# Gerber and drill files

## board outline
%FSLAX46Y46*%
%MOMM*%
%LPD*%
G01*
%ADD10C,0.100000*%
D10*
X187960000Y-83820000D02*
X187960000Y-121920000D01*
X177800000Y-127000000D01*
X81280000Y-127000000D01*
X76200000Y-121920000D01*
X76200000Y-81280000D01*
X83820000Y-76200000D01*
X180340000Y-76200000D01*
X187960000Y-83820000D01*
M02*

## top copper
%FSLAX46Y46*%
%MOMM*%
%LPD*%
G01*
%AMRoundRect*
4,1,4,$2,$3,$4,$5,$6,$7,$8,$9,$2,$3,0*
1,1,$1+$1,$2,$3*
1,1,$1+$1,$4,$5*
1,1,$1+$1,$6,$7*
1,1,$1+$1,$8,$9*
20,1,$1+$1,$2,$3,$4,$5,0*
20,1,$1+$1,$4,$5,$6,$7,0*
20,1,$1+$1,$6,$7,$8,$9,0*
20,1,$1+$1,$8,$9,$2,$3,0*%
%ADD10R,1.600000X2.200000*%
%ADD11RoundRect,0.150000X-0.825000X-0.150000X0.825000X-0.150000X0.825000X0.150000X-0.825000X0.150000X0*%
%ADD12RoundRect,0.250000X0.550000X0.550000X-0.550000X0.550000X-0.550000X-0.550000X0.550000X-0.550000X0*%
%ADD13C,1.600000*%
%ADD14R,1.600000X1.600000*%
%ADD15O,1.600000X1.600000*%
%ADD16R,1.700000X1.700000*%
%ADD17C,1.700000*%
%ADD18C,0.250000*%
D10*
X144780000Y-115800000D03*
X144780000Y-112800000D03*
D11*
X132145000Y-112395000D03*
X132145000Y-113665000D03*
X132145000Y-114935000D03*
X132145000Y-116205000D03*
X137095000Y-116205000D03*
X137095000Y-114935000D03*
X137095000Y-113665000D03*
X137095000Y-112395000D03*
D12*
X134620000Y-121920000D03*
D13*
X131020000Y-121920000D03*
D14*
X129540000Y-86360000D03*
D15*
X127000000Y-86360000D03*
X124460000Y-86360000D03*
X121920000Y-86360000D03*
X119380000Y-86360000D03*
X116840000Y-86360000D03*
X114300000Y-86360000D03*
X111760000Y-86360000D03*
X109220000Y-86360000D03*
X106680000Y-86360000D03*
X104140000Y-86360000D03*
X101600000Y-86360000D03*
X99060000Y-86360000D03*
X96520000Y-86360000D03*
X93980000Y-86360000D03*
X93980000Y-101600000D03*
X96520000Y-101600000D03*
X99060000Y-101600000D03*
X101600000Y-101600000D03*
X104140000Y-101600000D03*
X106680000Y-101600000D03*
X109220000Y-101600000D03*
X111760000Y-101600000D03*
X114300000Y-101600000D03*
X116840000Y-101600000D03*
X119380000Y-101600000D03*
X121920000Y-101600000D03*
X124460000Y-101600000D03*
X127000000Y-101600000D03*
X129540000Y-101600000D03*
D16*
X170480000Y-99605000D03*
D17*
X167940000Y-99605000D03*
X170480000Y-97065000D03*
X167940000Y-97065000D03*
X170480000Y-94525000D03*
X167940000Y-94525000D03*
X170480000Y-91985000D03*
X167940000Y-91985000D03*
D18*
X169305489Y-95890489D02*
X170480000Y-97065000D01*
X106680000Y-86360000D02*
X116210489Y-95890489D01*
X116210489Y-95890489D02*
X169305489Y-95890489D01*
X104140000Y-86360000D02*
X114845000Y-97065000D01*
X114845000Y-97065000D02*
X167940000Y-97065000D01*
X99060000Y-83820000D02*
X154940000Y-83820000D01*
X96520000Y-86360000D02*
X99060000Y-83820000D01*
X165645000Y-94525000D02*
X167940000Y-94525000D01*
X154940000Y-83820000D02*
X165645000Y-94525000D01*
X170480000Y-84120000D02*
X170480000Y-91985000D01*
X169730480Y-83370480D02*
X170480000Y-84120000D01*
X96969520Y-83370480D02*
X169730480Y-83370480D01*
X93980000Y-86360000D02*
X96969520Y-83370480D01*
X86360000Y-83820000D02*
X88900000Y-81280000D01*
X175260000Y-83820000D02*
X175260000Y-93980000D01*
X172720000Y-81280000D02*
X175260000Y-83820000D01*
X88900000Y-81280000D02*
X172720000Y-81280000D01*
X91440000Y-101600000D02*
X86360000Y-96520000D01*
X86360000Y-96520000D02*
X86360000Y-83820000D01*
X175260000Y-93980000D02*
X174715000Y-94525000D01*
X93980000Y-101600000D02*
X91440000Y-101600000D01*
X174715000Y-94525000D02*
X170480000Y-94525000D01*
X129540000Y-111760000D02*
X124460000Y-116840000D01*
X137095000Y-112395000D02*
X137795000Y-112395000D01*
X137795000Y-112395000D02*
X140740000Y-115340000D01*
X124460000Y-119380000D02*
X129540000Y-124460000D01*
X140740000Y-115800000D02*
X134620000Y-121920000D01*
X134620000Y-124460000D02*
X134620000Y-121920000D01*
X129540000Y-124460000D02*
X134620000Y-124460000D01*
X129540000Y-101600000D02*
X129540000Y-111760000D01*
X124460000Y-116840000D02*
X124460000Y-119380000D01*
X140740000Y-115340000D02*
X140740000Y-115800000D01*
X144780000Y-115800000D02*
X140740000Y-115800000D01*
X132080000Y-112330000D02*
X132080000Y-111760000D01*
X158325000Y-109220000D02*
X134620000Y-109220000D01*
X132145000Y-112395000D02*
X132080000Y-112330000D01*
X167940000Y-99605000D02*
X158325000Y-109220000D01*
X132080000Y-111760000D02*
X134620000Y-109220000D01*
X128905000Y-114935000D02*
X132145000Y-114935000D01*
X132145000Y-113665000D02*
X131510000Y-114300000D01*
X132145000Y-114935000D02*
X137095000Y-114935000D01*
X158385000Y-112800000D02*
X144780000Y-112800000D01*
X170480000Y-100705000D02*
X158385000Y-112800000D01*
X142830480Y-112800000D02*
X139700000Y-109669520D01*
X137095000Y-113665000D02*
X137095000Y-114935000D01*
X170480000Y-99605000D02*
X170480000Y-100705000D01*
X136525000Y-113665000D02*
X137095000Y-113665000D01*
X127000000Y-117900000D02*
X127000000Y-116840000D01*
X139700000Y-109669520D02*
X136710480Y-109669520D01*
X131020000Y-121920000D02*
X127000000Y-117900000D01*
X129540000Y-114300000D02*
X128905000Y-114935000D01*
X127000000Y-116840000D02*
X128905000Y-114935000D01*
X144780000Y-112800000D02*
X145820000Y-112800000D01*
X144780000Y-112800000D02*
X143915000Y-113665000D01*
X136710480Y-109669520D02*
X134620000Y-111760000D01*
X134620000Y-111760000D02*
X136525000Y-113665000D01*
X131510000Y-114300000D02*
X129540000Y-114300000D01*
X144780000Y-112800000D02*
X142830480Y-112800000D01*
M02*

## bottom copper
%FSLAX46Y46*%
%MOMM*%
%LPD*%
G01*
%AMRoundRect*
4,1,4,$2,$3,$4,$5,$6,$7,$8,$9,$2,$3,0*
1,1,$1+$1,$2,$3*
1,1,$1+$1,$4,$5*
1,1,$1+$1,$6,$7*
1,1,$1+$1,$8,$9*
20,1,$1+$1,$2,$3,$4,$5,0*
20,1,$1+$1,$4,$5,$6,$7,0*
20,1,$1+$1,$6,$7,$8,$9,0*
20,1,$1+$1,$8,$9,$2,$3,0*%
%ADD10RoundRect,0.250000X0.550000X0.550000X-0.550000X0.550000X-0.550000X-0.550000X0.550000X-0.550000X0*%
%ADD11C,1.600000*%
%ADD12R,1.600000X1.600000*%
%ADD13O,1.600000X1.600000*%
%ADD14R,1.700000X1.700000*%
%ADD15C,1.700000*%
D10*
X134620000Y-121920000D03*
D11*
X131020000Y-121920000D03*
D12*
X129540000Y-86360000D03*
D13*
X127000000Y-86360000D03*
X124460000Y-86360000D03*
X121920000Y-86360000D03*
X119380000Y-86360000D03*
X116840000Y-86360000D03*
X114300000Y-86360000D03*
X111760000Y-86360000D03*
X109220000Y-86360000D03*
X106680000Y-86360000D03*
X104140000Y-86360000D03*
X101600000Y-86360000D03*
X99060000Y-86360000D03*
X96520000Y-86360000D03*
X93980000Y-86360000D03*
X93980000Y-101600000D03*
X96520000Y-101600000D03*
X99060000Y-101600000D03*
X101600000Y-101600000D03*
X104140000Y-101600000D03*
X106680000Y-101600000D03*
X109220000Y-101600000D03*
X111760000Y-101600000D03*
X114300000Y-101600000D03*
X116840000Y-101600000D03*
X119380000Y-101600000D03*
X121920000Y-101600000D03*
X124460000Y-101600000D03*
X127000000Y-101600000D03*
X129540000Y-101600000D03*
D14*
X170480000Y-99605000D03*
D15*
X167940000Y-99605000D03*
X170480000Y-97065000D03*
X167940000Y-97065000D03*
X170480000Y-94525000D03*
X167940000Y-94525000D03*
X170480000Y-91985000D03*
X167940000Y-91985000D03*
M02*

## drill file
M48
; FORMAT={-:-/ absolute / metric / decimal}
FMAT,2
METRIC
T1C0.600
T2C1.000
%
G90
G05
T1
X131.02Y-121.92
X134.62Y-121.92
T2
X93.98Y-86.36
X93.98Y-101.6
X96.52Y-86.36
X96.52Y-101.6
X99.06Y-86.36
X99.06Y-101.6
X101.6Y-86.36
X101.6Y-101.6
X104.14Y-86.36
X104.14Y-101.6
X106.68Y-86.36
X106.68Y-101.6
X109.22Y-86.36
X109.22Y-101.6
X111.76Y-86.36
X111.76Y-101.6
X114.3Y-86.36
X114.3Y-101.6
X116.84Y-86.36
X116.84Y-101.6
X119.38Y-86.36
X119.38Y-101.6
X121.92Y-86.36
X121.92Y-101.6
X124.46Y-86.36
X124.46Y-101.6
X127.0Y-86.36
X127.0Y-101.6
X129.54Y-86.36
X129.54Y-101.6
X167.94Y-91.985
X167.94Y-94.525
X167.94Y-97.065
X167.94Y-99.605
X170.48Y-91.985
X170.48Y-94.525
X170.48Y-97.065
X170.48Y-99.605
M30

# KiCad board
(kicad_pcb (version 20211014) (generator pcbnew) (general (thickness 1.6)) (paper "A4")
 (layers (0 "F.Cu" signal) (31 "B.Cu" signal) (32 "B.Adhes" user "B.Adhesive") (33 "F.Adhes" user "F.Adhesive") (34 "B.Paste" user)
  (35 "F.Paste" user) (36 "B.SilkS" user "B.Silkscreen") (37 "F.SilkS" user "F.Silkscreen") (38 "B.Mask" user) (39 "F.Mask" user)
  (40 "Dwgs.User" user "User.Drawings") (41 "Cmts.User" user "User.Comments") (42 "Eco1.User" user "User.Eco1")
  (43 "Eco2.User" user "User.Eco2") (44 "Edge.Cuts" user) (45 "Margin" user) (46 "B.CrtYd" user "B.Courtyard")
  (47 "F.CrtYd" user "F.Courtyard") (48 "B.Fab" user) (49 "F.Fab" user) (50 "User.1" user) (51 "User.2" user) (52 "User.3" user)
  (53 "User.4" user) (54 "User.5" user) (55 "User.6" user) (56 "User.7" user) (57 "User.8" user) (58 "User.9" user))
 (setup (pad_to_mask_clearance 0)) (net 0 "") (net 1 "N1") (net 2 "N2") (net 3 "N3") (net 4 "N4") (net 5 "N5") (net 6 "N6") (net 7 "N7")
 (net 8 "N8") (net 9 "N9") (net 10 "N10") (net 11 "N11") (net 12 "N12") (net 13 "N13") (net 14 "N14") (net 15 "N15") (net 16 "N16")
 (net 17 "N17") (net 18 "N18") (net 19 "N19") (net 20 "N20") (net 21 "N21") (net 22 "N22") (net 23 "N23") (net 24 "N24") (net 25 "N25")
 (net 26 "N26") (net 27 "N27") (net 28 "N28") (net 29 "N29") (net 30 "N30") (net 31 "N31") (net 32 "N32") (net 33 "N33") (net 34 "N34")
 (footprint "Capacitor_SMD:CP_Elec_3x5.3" (layer "F.Cu") (at 144.78 114.3 90)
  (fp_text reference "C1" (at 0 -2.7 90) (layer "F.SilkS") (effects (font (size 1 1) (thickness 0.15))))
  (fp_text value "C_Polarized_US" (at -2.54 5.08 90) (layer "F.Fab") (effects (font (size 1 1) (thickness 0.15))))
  (pad "1" smd rect (at -1.5 0 90) (size 2.2 1.6) (layers "F.Cu" "F.Paste" "F.Mask") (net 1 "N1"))
  (pad "2" smd rect (at 1.5 0 90) (size 2.2 1.6) (layers "F.Cu" "F.Paste" "F.Mask") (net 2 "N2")))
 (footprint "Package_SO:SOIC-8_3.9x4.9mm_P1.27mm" (layer "F.Cu") (at 134.62 114.3)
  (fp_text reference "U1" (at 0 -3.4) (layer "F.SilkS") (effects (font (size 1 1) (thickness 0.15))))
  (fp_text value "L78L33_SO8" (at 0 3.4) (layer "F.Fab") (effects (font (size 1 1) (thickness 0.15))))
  (pad "1" smd roundrect (at -2.475 -1.905) (size 1.95 0.6) (layers "F.Cu" "F.Paste" "F.Mask") (roundrect_rratio 0.25) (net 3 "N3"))
  (pad "2" smd roundrect (at -2.475 -0.635) (size 1.95 0.6) (layers "F.Cu" "F.Paste" "F.Mask") (roundrect_rratio 0.25) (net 2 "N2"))
  (pad "3" smd roundrect (at -2.475 0.635) (size 1.95 0.6) (layers "F.Cu" "F.Paste" "F.Mask") (roundrect_rratio 0.25) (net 2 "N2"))
  (pad "4" smd roundrect (at -2.475 1.905) (size 1.95 0.6) (layers "F.Cu" "F.Paste" "F.Mask") (roundrect_rratio 0.25) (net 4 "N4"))
  (pad "5" smd roundrect (at 2.475 1.905) (size 1.95 0.6) (layers "F.Cu" "F.Paste" "F.Mask") (roundrect_rratio 0.25) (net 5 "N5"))
  (pad "6" smd roundrect (at 2.475 0.635) (size 1.95 0.6) (layers "F.Cu" "F.Paste" "F.Mask") (roundrect_rratio 0.25) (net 2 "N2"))
  (pad "7" smd roundrect (at 2.475 -0.635) (size 1.95 0.6) (layers "F.Cu" "F.Paste" "F.Mask") (roundrect_rratio 0.25) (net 2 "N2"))
  (pad "8" smd roundrect (at 2.475 -1.905) (size 1.95 0.6) (layers "F.Cu" "F.Paste" "F.Mask") (roundrect_rratio 0.25) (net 1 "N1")))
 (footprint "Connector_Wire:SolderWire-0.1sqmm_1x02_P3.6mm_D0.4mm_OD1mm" (layer "F.Cu") (at 134.62 121.92 180)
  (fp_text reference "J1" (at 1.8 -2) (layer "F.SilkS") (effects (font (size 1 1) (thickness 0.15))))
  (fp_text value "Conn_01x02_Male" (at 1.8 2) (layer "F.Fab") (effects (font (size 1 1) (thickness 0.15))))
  (pad "1" thru_hole roundrect (at 0 0 180) (size 1.6 1.6) (drill 0.6) (layers *.Cu *.Mask) (roundrect_rratio 0.15625) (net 1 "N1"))
  (pad "2" thru_hole circle (at 3.6 0 180) (size 1.6 1.6) (drill 0.6) (layers *.Cu *.Mask) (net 2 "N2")))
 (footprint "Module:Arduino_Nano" (layer "F.Cu") (at 129.54 86.36 -90)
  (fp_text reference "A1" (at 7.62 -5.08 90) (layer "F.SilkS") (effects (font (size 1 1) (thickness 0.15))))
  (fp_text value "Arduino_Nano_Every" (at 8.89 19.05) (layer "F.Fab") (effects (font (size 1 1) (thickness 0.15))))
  (pad "1" thru_hole rect (at 0 0 270) (size 1.6 1.6) (drill 1) (layers *.Cu *.Mask) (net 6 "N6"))
  (pad "2" thru_hole oval (at 0 2.54 270) (size 1.6 1.6) (drill 1) (layers *.Cu *.Mask) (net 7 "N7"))
  (pad "3" thru_hole oval (at 0 5.08 270) (size 1.6 1.6) (drill 1) (layers *.Cu *.Mask) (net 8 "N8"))
  (pad "4" thru_hole oval (at 0 7.62 270) (size 1.6 1.6) (drill 1) (layers *.Cu *.Mask) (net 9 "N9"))
  (pad "5" thru_hole oval (at 0 10.16 270) (size 1.6 1.6) (drill 1) (layers *.Cu *.Mask) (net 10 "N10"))
  (pad "6" thru_hole oval (at 0 12.7 270) (size 1.6 1.6) (drill 1) (layers *.Cu *.Mask) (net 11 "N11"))
  (pad "7" thru_hole oval (at 0 15.24 270) (size 1.6 1.6) (drill 1) (layers *.Cu *.Mask) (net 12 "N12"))
  (pad "8" thru_hole oval (at 0 17.78 270) (size 1.6 1.6) (drill 1) (layers *.Cu *.Mask) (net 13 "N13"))
  (pad "9" thru_hole oval (at 0 20.32 270) (size 1.6 1.6) (drill 1) (layers *.Cu *.Mask) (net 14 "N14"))
  (pad "10" thru_hole oval (at 0 22.86 270) (size 1.6 1.6) (drill 1) (layers *.Cu *.Mask) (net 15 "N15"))
  (pad "11" thru_hole oval (at 0 25.4 270) (size 1.6 1.6) (drill 1) (layers *.Cu *.Mask) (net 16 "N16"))
  (pad "12" thru_hole oval (at 0 27.94 270) (size 1.6 1.6) (drill 1) (layers *.Cu *.Mask) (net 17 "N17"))
  (pad "13" thru_hole oval (at 0 30.48 270) (size 1.6 1.6) (drill 1) (layers *.Cu *.Mask) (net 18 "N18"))
  (pad "14" thru_hole oval (at 0 33.02 270) (size 1.6 1.6) (drill 1) (layers *.Cu *.Mask) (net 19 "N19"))
  (pad "15" thru_hole oval (at 0 35.56 270) (size 1.6 1.6) (drill 1) (layers *.Cu *.Mask) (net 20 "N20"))
  (pad "16" thru_hole oval (at 15.24 35.56 270) (size 1.6 1.6) (drill 1) (layers *.Cu *.Mask) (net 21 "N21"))
  (pad "17" thru_hole oval (at 15.24 33.02 270) (size 1.6 1.6) (drill 1) (layers *.Cu *.Mask) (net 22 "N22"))
  (pad "18" thru_hole oval (at 15.24 30.48 270) (size 1.6 1.6) (drill 1) (layers *.Cu *.Mask) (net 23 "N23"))
  (pad "19" thru_hole oval (at 15.24 27.94 270) (size 1.6 1.6) (drill 1) (layers *.Cu *.Mask) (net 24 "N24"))
  (pad "20" thru_hole oval (at 15.24 25.4 270) (size 1.6 1.6) (drill 1) (layers *.Cu *.Mask) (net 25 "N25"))
  (pad "21" thru_hole oval (at 15.24 22.86 270) (size 1.6 1.6) (drill 1) (layers *.Cu *.Mask) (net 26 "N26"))
  (pad "22" thru_hole oval (at 15.24 20.32 270) (size 1.6 1.6) (drill 1) (layers *.Cu *.Mask) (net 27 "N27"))
  (pad "23" thru_hole oval (at 15.24 17.78 270) (size 1.6 1.6) (drill 1) (layers *.Cu *.Mask) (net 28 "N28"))
  (pad "24" thru_hole oval (at 15.24 15.24 270) (size 1.6 1.6) (drill 1) (layers *.Cu *.Mask) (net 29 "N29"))
  (pad "25" thru_hole oval (at 15.24 12.7 270) (size 1.6 1.6) (drill 1) (layers *.Cu *.Mask) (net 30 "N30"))
  (pad "26" thru_hole oval (at 15.24 10.16 270) (size 1.6 1.6) (drill 1) (layers *.Cu *.Mask) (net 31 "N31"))
  (pad "27" thru_hole oval (at 15.24 7.62 270) (size 1.6 1.6) (drill 1) (layers *.Cu *.Mask) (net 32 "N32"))
  (pad "28" thru_hole oval (at 15.24 5.08 270) (size 1.6 1.6) (drill 1) (layers *.Cu *.Mask) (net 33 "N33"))
  (pad "29" thru_hole oval (at 15.24 2.54 270) (size 1.6 1.6) (drill 1) (layers *.Cu *.Mask) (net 9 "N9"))
  (pad "30" thru_hole oval (at 15.24 0 270) (size 1.6 1.6) (drill 1) (layers *.Cu *.Mask) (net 1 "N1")))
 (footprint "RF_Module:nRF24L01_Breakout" (layer "F.Cu") (at 170.48 99.605 180)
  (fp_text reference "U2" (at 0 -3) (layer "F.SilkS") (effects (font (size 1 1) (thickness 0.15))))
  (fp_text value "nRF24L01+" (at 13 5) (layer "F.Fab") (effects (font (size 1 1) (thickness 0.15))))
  (pad "1" thru_hole rect (at 0 0 180) (size 1.7 1.7) (drill 1) (layers *.Cu *.Mask) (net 2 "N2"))
  (pad "2" thru_hole circle (at 2.54 0 180) (size 1.7 1.7) (drill 1) (layers *.Cu *.Mask) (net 3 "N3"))
  (pad "3" thru_hole circle (at 0 2.54 180) (size 1.7 1.7) (drill 1) (layers *.Cu *.Mask) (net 15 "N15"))
  (pad "4" thru_hole circle (at 2.54 2.54 180) (size 1.7 1.7) (drill 1) (layers *.Cu *.Mask) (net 16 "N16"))
  (pad "5" thru_hole circle (at 0 5.08 180) (size 1.7 1.7) (drill 1) (layers *.Cu *.Mask) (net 21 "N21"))
  (pad "6" thru_hole circle (at 2.54 5.08 180) (size 1.7 1.7) (drill 1) (layers *.Cu *.Mask) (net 19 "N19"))
  (pad "7" thru_hole circle (at 0 7.62 180) (size 1.7 1.7) (drill 1) (layers *.Cu *.Mask) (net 20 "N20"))
  (pad "8" thru_hole circle (at 2.54 7.62 180) (size 1.7 1.7) (drill 1) (layers *.Cu *.Mask) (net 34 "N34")))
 (gr_poly
  (pts (xy 187.96 83.82) (xy 187.96 121.92) (xy 177.8 127) (xy 81.28 127) (xy 76.2 121.92) (xy 76.2 81.28) (xy 83.82 76.2) (xy 180.34 76.2))
  (layer "Edge.Cuts") (width 0.1) (fill none))
 (segment (start 169.305489 95.890489) (end 170.48 97.065) (width 0.25) (layer "F.Cu") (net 15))
 (segment (start 106.68 86.36) (end 116.210489 95.890489) (width 0.25) (layer "F.Cu") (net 15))
 (segment (start 116.210489 95.890489) (end 169.305489 95.890489) (width 0.25) (layer "F.Cu") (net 15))
 (segment (start 104.14 86.36) (end 114.845 97.065) (width 0.25) (layer "F.Cu") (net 16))
 (segment (start 114.845 97.065) (end 167.94 97.065) (width 0.25) (layer "F.Cu") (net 16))
 (segment (start 99.06 83.82) (end 154.94 83.82) (width 0.25) (layer "F.Cu") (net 19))
 (segment (start 96.52 86.36) (end 99.06 83.82) (width 0.25) (layer "F.Cu") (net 19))
 (segment (start 165.645 94.525) (end 167.94 94.525) (width 0.25) (layer "F.Cu") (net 19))
 (segment (start 154.94 83.82) (end 165.645 94.525) (width 0.25) (layer "F.Cu") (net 19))
 (segment (start 170.48 84.12) (end 170.48 91.985) (width 0.25) (layer "F.Cu") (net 20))
 (segment (start 169.73048 83.37048) (end 170.48 84.12) (width 0.25) (layer "F.Cu") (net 20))
 (segment (start 96.96952 83.37048) (end 169.73048 83.37048) (width 0.25) (layer "F.Cu") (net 20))
 (segment (start 93.98 86.36) (end 96.96952 83.37048) (width 0.25) (layer "F.Cu") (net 20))
 (segment (start 86.36 83.82) (end 88.9 81.28) (width 0.25) (layer "F.Cu") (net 21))
 (segment (start 175.26 83.82) (end 175.26 93.98) (width 0.25) (layer "F.Cu") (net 21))
 (segment (start 172.72 81.28) (end 175.26 83.82) (width 0.25) (layer "F.Cu") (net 21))
 (segment (start 88.9 81.28) (end 172.72 81.28) (width 0.25) (layer "F.Cu") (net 21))
 (segment (start 91.44 101.6) (end 86.36 96.52) (width 0.25) (layer "F.Cu") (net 21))
 (segment (start 86.36 96.52) (end 86.36 83.82) (width 0.25) (layer "F.Cu") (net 21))
 (segment (start 175.26 93.98) (end 174.715 94.525) (width 0.25) (layer "F.Cu") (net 21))
 (segment (start 93.98 101.6) (end 91.44 101.6) (width 0.25) (layer "F.Cu") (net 21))
 (segment (start 174.715 94.525) (end 170.48 94.525) (width 0.25) (layer "F.Cu") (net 21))
 (segment (start 129.54 111.76) (end 124.46 116.84) (width 0.25) (layer "F.Cu") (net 1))
 (segment (start 137.095 112.395) (end 137.795 112.395) (width 0.25) (layer "F.Cu") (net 1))
 (segment (start 137.795 112.395) (end 140.74 115.34) (width 0.25) (layer "F.Cu") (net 1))
 (segment (start 124.46 119.38) (end 129.54 124.46) (width 0.25) (layer "F.Cu") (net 1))
 (segment (start 140.74 115.8) (end 134.62 121.92) (width 0.25) (layer "F.Cu") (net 1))
 (segment (start 134.62 124.46) (end 134.62 121.92) (width 0.25) (layer "F.Cu") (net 1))
 (segment (start 129.54 124.46) (end 134.62 124.46) (width 0.25) (layer "F.Cu") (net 1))
 (segment (start 129.54 101.6) (end 129.54 111.76) (width 0.25) (layer "F.Cu") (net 1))
 (segment (start 124.46 116.84) (end 124.46 119.38) (width 0.25) (layer "F.Cu") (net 1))
 (segment (start 140.74 115.34) (end 140.74 115.8) (width 0.25) (layer "F.Cu") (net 1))
 (segment (start 144.78 115.8) (end 140.74 115.8) (width 0.25) (layer "F.Cu") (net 1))
 (segment (start 132.08 112.33) (end 132.08 111.76) (width 0.25) (layer "F.Cu") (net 3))
 (segment (start 158.325 109.22) (end 134.62 109.22) (width 0.25) (layer "F.Cu") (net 3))
 (segment (start 132.145 112.395) (end 132.08 112.33) (width 0.25) (layer "F.Cu") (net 3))
 (segment (start 167.94 99.605) (end 158.325 109.22) (width 0.25) (layer "F.Cu") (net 3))
 (segment (start 132.08 111.76) (end 134.62 109.22) (width 0.25) (layer "F.Cu") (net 3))
 (segment (start 128.905 114.935) (end 132.145 114.935) (width 0.25) (layer "F.Cu") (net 2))
 (segment (start 132.145 113.665) (end 131.51 114.3) (width 0.25) (layer "F.Cu") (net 2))
 (segment (start 132.145 114.935) (end 137.095 114.935) (width 0.25) (layer "F.Cu") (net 2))
 (segment (start 158.385 112.8) (end 144.78 112.8) (width 0.25) (layer "F.Cu") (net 2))
 (segment (start 170.48 100.705) (end 158.385 112.8) (width 0.25) (layer "F.Cu") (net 2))
 (segment (start 142.83048 112.8) (end 139.7 109.66952) (width 0.25) (layer "F.Cu") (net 2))
 (segment (start 137.095 113.665) (end 137.095 114.935) (width 0.25) (layer "F.Cu") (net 2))
 (segment (start 170.48 99.605) (end 170.48 100.705) (width 0.25) (layer "F.Cu") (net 2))
 (segment (start 136.525 113.665) (end 137.095 113.665) (width 0.25) (layer "F.Cu") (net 2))
 (segment (start 127 117.9) (end 127 116.84) (width 0.25) (layer "F.Cu") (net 2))
 (segment (start 139.7 109.66952) (end 136.71048 109.66952) (width 0.25) (layer "F.Cu") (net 2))
 (segment (start 131.02 121.92) (end 127 117.9) (width 0.25) (layer "F.Cu") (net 2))
 (segment (start 129.54 114.3) (end 128.905 114.935) (width 0.25) (layer "F.Cu") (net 2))
 (segment (start 127 116.84) (end 128.905 114.935) (width 0.25) (layer "F.Cu") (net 2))
 (segment (start 144.78 112.8) (end 145.82 112.8) (width 0.25) (layer "F.Cu") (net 2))
 (segment (start 144.78 112.8) (end 143.915 113.665) (width 0.25) (layer "F.Cu") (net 2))
 (segment (start 136.71048 109.66952) (end 134.62 111.76) (width 0.25) (layer "F.Cu") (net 2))
 (segment (start 134.62 111.76) (end 136.525 113.665) (width 0.25) (layer "F.Cu") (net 2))
 (segment (start 131.51 114.3) (end 129.54 114.3) (width 0.25) (layer "F.Cu") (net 2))
 (segment (start 144.78 112.8) (end 142.83048 112.8) (width 0.25) (layer "F.Cu") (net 2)))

